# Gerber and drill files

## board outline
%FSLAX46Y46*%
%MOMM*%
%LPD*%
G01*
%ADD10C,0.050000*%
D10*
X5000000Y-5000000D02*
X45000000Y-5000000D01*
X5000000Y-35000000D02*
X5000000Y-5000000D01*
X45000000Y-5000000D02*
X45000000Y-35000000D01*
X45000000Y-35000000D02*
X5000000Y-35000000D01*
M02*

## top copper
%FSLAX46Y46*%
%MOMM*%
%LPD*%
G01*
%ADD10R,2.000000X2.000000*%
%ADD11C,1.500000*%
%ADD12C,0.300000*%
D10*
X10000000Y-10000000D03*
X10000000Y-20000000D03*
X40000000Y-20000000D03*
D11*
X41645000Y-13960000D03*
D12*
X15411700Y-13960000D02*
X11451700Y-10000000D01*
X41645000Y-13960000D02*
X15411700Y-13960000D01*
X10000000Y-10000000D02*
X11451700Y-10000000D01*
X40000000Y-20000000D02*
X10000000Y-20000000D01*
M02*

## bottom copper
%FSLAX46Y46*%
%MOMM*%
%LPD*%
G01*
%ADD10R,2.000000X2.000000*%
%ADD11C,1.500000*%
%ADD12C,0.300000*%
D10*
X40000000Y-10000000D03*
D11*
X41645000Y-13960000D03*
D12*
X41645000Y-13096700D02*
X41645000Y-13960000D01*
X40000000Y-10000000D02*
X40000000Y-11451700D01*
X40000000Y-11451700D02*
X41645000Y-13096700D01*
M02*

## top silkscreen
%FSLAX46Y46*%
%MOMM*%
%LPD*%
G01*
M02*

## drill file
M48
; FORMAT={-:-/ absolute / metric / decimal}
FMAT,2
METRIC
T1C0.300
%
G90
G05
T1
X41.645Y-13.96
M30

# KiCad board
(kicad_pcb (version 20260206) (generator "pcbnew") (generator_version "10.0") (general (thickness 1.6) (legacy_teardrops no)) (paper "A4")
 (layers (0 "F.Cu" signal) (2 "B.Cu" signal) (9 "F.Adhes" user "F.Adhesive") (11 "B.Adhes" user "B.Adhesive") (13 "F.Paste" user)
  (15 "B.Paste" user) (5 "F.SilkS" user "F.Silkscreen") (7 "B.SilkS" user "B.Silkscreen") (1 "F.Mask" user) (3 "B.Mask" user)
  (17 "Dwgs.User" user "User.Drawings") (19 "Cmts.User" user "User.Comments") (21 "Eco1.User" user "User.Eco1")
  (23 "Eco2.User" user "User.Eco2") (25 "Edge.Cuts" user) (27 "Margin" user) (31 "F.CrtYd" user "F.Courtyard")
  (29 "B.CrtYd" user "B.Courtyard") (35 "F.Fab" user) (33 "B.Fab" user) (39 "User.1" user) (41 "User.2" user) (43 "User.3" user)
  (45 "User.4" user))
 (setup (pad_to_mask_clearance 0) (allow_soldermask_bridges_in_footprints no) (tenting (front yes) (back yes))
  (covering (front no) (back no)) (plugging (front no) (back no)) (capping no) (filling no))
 (gr_line (start 5 5) (end 45 5) (stroke (width 0.05) (type default)) (layer "Edge.Cuts"))
 (gr_line (start 5 35) (end 5 5) (stroke (width 0.05) (type default)) (layer "Edge.Cuts"))
 (gr_line (start 45 5) (end 45 35) (stroke (width 0.05) (type default)) (layer "Edge.Cuts"))
 (gr_line (start 45 35) (end 5 35) (stroke (width 0.05) (type default)) (layer "Edge.Cuts"))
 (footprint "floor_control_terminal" (layer "F.Cu") (at 10 10)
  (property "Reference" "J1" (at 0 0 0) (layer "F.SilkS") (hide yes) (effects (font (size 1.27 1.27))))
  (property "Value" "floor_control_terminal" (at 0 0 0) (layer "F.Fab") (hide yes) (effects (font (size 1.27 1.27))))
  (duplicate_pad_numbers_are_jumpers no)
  (pad "1" smd rect (at 0 0) (size 2 2) (layers "F.Cu" "F.Paste" "F.Mask") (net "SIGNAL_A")))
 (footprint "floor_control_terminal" (layer "B.Cu") (at 40 10)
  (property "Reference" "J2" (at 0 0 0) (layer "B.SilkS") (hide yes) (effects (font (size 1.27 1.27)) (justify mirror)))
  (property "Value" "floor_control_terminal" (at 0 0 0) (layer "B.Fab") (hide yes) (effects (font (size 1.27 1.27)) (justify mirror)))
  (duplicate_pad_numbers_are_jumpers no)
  (pad "1" smd rect (at 0 0) (size 2 2) (layers "B.Cu" "B.Paste" "B.Mask") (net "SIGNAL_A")))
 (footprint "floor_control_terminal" (layer "F.Cu") (at 10 20)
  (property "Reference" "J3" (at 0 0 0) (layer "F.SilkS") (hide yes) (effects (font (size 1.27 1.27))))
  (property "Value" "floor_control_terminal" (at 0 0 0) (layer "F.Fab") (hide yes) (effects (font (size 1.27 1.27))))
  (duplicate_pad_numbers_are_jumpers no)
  (pad "1" smd rect (at 0 0) (size 2 2) (layers "F.Cu" "F.Paste" "F.Mask") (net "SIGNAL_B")))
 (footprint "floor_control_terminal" (layer "F.Cu") (at 40 20)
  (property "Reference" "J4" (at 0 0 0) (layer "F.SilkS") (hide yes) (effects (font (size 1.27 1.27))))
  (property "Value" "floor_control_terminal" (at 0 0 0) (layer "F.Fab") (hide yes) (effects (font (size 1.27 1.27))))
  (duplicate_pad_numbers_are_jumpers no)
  (pad "1" smd rect (at 0 0) (size 2 2) (layers "F.Cu" "F.Paste" "F.Mask") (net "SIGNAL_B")))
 (segment (start 15.4117 13.96) (end 11.4517 10) (width 0.3) (layer "F.Cu") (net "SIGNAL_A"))
 (segment (start 41.645 13.96) (end 15.4117 13.96) (width 0.3) (layer "F.Cu") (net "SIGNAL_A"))
 (segment (start 10 10) (end 11.4517 10) (width 0.3) (layer "F.Cu") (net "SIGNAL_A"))
 (via (at 41.645 13.96) (size 1.5) (drill 0.3) (layers "F.Cu" "B.Cu") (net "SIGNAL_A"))
 (segment (start 41.645 13.0967) (end 41.645 13.96) (width 0.3) (layer "B.Cu") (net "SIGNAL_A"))
 (segment (start 40 10) (end 40 11.4517) (width 0.3) (layer "B.Cu") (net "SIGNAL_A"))
 (segment (start 40 11.4517) (end 41.645 13.0967) (width 0.3) (layer "B.Cu") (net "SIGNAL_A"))
 (segment (start 40 20) (end 10 20) (width 0.3) (layer "F.Cu") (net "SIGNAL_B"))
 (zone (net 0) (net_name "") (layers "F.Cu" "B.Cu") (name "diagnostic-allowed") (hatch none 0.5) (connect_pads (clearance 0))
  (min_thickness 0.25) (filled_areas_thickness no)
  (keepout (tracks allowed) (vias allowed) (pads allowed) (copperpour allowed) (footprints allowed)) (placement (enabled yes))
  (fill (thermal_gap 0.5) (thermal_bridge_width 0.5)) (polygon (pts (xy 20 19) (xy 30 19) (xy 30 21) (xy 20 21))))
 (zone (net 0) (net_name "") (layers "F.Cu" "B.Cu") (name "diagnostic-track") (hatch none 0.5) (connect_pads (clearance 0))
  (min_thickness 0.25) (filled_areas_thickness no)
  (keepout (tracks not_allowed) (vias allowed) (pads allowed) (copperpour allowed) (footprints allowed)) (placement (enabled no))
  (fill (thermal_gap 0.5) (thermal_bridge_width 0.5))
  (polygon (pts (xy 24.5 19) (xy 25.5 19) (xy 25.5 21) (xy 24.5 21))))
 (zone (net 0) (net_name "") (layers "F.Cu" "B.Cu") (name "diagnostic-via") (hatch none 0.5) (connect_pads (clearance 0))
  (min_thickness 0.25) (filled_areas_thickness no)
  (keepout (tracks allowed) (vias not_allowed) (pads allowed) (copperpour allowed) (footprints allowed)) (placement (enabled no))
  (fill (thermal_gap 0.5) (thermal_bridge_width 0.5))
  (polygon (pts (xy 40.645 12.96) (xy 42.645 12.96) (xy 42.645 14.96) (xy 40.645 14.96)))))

